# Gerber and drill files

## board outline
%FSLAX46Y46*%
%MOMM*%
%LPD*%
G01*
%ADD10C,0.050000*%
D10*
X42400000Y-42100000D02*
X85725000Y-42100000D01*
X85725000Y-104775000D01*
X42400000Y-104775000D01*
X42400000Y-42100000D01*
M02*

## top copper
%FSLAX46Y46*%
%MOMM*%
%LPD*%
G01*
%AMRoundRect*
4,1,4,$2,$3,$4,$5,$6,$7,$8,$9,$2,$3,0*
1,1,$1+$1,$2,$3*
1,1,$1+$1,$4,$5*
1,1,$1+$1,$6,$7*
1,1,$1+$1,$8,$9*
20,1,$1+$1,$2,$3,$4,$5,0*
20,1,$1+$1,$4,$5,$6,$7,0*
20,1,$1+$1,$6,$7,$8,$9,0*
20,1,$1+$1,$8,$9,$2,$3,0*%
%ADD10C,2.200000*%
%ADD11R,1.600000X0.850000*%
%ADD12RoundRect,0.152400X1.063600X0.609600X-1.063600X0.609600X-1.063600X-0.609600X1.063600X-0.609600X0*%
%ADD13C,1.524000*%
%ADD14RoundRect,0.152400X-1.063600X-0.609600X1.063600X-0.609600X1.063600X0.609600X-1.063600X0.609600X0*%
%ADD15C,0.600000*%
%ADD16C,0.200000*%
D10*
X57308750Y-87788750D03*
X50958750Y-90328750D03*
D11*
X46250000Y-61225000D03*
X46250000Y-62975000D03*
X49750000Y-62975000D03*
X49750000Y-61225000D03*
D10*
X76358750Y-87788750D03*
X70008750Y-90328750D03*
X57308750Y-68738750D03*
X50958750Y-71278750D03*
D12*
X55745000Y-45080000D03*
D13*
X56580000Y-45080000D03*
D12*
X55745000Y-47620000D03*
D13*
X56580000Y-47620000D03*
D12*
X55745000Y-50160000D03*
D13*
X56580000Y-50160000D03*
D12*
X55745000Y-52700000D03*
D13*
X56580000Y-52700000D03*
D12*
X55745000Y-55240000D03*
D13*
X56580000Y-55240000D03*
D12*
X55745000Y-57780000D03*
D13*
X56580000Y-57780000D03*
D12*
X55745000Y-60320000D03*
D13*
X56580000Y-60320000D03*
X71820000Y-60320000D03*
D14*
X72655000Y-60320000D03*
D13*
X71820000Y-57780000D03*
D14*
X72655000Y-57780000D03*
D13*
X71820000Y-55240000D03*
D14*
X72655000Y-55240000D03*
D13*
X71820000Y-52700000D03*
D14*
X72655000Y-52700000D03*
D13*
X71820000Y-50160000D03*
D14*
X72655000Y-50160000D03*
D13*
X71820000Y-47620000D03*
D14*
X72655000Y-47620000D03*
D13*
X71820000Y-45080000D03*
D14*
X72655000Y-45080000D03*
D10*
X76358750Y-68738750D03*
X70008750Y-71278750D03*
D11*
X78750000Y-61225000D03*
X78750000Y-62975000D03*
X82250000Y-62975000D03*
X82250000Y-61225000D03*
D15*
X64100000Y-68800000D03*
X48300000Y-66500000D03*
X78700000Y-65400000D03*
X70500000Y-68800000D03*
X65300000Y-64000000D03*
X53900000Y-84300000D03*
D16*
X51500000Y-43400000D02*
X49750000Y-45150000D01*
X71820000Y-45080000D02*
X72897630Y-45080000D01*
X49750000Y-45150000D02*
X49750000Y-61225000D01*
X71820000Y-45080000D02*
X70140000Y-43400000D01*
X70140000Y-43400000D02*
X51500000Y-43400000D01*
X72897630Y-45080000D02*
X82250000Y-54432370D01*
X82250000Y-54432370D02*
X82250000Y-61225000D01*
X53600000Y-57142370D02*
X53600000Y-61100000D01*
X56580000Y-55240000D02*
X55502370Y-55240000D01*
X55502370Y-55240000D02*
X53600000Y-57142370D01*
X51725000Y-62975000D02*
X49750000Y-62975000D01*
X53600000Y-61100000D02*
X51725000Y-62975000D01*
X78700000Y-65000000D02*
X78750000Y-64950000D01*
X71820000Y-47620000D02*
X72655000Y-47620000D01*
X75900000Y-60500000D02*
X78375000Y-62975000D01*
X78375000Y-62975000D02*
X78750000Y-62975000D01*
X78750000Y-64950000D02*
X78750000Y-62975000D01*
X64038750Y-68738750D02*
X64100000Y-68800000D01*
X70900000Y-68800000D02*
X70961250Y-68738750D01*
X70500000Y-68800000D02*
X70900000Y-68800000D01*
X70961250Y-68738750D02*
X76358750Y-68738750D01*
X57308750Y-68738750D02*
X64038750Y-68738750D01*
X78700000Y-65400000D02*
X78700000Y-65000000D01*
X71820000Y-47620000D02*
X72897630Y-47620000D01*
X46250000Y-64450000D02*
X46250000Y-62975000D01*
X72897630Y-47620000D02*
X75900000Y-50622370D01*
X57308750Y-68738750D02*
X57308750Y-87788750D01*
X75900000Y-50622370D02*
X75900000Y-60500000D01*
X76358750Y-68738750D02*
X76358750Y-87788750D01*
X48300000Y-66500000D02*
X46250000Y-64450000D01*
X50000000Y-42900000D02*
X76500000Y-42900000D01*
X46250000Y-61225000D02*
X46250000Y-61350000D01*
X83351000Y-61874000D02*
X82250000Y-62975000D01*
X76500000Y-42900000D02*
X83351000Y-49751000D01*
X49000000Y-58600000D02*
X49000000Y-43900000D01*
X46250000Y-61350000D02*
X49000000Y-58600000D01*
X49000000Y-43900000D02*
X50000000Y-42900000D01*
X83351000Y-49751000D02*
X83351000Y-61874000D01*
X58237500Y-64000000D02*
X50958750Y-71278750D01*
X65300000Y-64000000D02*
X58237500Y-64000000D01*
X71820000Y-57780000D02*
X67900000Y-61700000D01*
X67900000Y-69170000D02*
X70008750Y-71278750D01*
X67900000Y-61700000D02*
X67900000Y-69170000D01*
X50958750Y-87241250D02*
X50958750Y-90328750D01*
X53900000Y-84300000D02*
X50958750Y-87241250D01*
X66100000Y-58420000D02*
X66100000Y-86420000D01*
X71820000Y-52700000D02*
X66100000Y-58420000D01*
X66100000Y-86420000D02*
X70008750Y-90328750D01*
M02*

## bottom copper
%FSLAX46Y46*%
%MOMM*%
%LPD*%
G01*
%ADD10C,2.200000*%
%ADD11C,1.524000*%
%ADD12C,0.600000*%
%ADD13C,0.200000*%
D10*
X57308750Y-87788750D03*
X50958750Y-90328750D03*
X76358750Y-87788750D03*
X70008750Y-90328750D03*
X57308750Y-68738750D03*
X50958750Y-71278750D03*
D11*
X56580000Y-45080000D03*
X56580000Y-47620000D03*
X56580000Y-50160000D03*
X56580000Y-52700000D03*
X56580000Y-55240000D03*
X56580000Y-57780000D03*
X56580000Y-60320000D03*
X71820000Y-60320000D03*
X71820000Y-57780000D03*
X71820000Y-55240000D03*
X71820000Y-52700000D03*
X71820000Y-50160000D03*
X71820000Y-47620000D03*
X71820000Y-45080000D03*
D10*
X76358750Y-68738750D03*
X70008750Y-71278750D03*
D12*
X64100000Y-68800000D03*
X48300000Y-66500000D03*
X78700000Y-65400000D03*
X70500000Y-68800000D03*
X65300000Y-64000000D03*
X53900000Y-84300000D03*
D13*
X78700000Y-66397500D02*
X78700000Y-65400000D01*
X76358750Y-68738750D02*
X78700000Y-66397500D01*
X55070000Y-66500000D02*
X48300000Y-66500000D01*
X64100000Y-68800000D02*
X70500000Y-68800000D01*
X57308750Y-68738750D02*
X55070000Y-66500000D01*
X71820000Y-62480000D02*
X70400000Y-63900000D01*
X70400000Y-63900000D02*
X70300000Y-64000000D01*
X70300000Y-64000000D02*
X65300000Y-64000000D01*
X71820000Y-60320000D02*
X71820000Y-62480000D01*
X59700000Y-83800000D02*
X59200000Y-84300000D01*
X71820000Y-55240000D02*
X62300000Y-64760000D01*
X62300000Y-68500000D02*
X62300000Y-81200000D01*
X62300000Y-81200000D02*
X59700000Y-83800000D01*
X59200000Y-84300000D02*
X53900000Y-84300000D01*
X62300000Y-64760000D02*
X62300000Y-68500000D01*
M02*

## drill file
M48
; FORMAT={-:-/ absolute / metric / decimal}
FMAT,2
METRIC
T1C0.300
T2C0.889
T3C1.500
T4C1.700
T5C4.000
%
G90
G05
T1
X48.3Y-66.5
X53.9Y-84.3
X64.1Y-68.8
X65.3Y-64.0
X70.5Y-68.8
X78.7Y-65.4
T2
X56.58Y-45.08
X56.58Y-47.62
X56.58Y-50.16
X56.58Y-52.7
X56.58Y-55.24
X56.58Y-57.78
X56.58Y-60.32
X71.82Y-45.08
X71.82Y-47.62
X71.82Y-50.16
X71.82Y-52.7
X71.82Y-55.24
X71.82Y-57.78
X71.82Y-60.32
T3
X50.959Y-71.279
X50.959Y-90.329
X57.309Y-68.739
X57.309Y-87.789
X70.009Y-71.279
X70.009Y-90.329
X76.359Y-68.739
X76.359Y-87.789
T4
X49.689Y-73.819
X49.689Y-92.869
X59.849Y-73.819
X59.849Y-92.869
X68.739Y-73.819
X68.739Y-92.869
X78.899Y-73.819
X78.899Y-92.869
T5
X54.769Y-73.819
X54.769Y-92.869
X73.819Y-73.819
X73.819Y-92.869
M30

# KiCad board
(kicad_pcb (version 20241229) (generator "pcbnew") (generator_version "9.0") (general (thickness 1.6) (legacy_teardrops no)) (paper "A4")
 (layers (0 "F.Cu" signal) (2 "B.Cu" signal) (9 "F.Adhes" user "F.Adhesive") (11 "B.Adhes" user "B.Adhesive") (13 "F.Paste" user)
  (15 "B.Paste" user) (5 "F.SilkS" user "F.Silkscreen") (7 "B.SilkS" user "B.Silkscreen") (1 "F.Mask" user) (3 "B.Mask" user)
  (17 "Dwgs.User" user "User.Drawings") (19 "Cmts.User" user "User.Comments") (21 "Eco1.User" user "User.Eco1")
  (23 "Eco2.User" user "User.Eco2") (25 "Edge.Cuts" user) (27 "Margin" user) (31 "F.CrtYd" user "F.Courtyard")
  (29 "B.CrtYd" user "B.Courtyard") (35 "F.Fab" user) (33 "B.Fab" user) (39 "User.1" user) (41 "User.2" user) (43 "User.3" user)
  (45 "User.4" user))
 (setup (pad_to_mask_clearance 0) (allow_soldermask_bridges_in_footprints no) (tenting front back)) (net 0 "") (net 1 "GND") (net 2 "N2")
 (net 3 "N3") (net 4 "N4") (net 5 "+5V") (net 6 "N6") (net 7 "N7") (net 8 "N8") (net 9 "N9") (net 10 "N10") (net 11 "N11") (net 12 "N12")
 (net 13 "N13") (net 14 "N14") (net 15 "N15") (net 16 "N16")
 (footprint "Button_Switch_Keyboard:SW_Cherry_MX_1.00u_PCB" (layer "F.Cu") (at 57.30875 87.78875)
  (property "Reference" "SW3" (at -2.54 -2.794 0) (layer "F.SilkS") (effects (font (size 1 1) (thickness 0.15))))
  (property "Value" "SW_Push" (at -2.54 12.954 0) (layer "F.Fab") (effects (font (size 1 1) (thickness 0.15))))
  (pad "" np_thru_hole circle (at -7.62 5.08) (size 1.7 1.7) (drill 1.7) (layers "*.Cu" "*.Mask"))
  (pad "" np_thru_hole circle (at -2.54 5.08) (size 4 4) (drill 4) (layers "*.Cu" "*.Mask"))
  (pad "" np_thru_hole circle (at 2.54 5.08) (size 1.7 1.7) (drill 1.7) (layers "*.Cu" "*.Mask"))
  (pad "1" thru_hole circle (at 0 0) (size 2.2 2.2) (drill 1.5) (layers "*.Cu" "*.Mask") (remove_unused_layers no) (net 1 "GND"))
  (pad "2" thru_hole circle (at -6.35 2.54) (size 2.2 2.2) (drill 1.5) (layers "*.Cu" "*.Mask") (remove_unused_layers no) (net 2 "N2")))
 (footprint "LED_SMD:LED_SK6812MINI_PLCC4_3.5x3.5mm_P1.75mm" (layer "F.Cu") (at 48 62.1)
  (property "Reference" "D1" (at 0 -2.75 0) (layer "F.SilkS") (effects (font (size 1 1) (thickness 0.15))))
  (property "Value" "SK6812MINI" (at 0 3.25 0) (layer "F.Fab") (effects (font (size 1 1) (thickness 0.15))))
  (pad "1" smd rect (at -1.75 -0.875) (size 1.6 0.85) (layers "F.Cu" "F.Mask" "F.Paste") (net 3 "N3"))
  (pad "2" smd rect (at -1.75 0.875) (size 1.6 0.85) (layers "F.Cu" "F.Mask" "F.Paste") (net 1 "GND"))
  (pad "3" smd rect (at 1.75 0.875) (size 1.6 0.85) (layers "F.Cu" "F.Mask" "F.Paste") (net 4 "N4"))
  (pad "4" smd rect (at 1.75 -0.875) (size 1.6 0.85) (layers "F.Cu" "F.Mask" "F.Paste") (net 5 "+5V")))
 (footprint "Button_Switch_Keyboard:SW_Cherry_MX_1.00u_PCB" (layer "F.Cu") (at 76.35875 87.78875)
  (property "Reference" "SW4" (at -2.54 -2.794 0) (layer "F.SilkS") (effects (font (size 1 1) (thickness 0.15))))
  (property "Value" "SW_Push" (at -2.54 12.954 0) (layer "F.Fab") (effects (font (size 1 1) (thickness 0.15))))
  (pad "" np_thru_hole circle (at -7.62 5.08) (size 1.7 1.7) (drill 1.7) (layers "*.Cu" "*.Mask"))
  (pad "" np_thru_hole circle (at -2.54 5.08) (size 4 4) (drill 4) (layers "*.Cu" "*.Mask"))
  (pad "" np_thru_hole circle (at 2.54 5.08) (size 1.7 1.7) (drill 1.7) (layers "*.Cu" "*.Mask"))
  (pad "1" thru_hole circle (at 0 0) (size 2.2 2.2) (drill 1.5) (layers "*.Cu" "*.Mask") (remove_unused_layers no) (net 1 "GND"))
  (pad "2" thru_hole circle (at -6.35 2.54) (size 2.2 2.2) (drill 1.5) (layers "*.Cu" "*.Mask") (remove_unused_layers no) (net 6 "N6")))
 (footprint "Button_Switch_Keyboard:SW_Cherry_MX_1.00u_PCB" (layer "F.Cu") (at 57.30875 68.73875)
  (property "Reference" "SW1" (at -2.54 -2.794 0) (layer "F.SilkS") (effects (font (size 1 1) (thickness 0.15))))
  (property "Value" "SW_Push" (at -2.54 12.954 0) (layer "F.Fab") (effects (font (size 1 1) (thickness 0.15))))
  (pad "" np_thru_hole circle (at -7.62 5.08) (size 1.7 1.7) (drill 1.7) (layers "*.Cu" "*.Mask"))
  (pad "" np_thru_hole circle (at -2.54 5.08) (size 4 4) (drill 4) (layers "*.Cu" "*.Mask"))
  (pad "" np_thru_hole circle (at 2.54 5.08) (size 1.7 1.7) (drill 1.7) (layers "*.Cu" "*.Mask"))
  (pad "1" thru_hole circle (at 0 0) (size 2.2 2.2) (drill 1.5) (layers "*.Cu" "*.Mask") (remove_unused_layers no) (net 1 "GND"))
  (pad "2" thru_hole circle (at -6.35 2.54) (size 2.2 2.2) (drill 1.5) (layers "*.Cu" "*.Mask") (remove_unused_layers no) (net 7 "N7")))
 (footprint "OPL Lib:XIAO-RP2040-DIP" (layer "F.Cu") (at 64.2 52.7)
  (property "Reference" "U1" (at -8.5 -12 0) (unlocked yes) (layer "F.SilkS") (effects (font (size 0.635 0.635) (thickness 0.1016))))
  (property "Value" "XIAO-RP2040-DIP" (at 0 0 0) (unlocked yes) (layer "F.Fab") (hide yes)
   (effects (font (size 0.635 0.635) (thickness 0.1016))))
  (pad "1" smd roundrect (at -8.455 -7.62 180) (size 2.432 1.524) (layers "F.Cu" "F.Mask") (roundrect_rratio 0.1) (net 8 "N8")
   (thermal_bridge_angle 45))
  (pad "1" thru_hole circle (at -7.62 -7.62 180) (size 1.524 1.524) (drill 0.889) (layers "*.Cu" "*.Mask") (remove_unused_layers no)
   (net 8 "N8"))
  (pad "2" smd roundrect (at -8.455 -5.08 180) (size 2.432 1.524) (layers "F.Cu" "F.Mask") (roundrect_rratio 0.1) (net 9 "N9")
   (thermal_bridge_angle 45))
  (pad "2" thru_hole circle (at -7.62 -5.08 180) (size 1.524 1.524) (drill 0.889) (layers "*.Cu" "*.Mask") (remove_unused_layers no)
   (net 9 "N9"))
  (pad "3" smd roundrect (at -8.455 -2.54 180) (size 2.432 1.524) (layers "F.Cu" "F.Mask") (roundrect_rratio 0.1) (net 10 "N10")
   (thermal_bridge_angle 45))
  (pad "3" thru_hole circle (at -7.62 -2.54 180) (size 1.524 1.524) (drill 0.889) (layers "*.Cu" "*.Mask") (remove_unused_layers no)
   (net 10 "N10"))
  (pad "4" smd roundrect (at -8.455 0 180) (size 2.432 1.524) (layers "F.Cu" "F.Mask") (roundrect_rratio 0.1) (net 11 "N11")
   (thermal_bridge_angle 45))
  (pad "4" thru_hole circle (at -7.62 0 180) (size 1.524 1.524) (drill 0.889) (layers "*.Cu" "*.Mask") (remove_unused_layers no)
   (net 11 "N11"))
  (pad "5" smd roundrect (at -8.455 2.54 180) (size 2.432 1.524) (layers "F.Cu" "F.Mask") (roundrect_rratio 0.1) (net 4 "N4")
   (thermal_bridge_angle 45))
  (pad "5" thru_hole circle (at -7.62 2.54 180) (size 1.524 1.524) (drill 0.889) (layers "*.Cu" "*.Mask") (remove_unused_layers no)
   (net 4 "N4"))
  (pad "6" smd roundrect (at -8.455 5.08 180) (size 2.432 1.524) (layers "F.Cu" "F.Mask") (roundrect_rratio 0.1) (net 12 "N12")
   (thermal_bridge_angle 45))
  (pad "6" thru_hole circle (at -7.62 5.08 180) (size 1.524 1.524) (drill 0.889) (layers "*.Cu" "*.Mask") (remove_unused_layers no)
   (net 12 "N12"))
  (pad "7" smd roundrect (at -8.455 7.62 180) (size 2.432 1.524) (layers "F.Cu" "F.Mask") (roundrect_rratio 0.1) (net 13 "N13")
   (thermal_bridge_angle 45))
  (pad "7" thru_hole circle (at -7.62 7.62 180) (size 1.524 1.524) (drill 0.889) (layers "*.Cu" "*.Mask") (remove_unused_layers no)
   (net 13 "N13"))
  (pad "8" thru_hole circle (at 7.62 7.62) (size 1.524 1.524) (drill 0.889) (layers "*.Cu" "*.Mask") (remove_unused_layers no) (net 7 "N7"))
  (pad "8" smd roundrect (at 8.455 7.62) (size 2.432 1.524) (layers "F.Cu" "F.Mask") (roundrect_rratio 0.1) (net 7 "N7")
   (thermal_bridge_angle 45))
  (pad "9" thru_hole circle (at 7.62 5.08) (size 1.524 1.524) (drill 0.889) (layers "*.Cu" "*.Mask") (remove_unused_layers no)
   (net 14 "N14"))
  (pad "9" smd roundrect (at 8.455 5.08) (size 2.432 1.524) (layers "F.Cu" "F.Mask") (roundrect_rratio 0.1) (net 14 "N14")
   (thermal_bridge_angle 45))
  (pad "10" thru_hole circle (at 7.62 2.54) (size 1.524 1.524) (drill 0.889) (layers "*.Cu" "*.Mask") (remove_unused_layers no) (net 2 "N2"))
  (pad "10" smd roundrect (at 8.455 2.54) (size 2.432 1.524) (layers "F.Cu" "F.Mask") (roundrect_rratio 0.1) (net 2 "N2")
   (thermal_bridge_angle 45))
  (pad "11" thru_hole circle (at 7.62 0) (size 1.524 1.524) (drill 0.889) (layers "*.Cu" "*.Mask") (remove_unused_layers no) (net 6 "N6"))
  (pad "11" smd roundrect (at 8.455 0) (size 2.432 1.524) (layers "F.Cu" "F.Mask") (roundrect_rratio 0.1) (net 6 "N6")
   (thermal_bridge_angle 45))
  (pad "12" thru_hole circle (at 7.62 -2.54) (size 1.524 1.524) (drill 0.889) (layers "*.Cu" "*.Mask") (remove_unused_layers no)
   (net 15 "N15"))
  (pad "12" smd roundrect (at 8.455 -2.54) (size 2.432 1.524) (layers "F.Cu" "F.Mask") (roundrect_rratio 0.1) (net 15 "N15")
   (thermal_bridge_angle 45))
  (pad "13" thru_hole circle (at 7.62 -5.08) (size 1.524 1.524) (drill 0.889) (layers "*.Cu" "*.Mask") (remove_unused_layers no)
   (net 1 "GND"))
  (pad "13" smd roundrect (at 8.455 -5.08) (size 2.432 1.524) (layers "F.Cu" "F.Mask") (roundrect_rratio 0.1) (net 1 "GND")
   (thermal_bridge_angle 45))
  (pad "14" thru_hole circle (at 7.62 -7.62) (size 1.524 1.524) (drill 0.889) (layers "*.Cu" "*.Mask") (remove_unused_layers no)
   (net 5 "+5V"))
  (pad "14" smd roundrect (at 8.455 -7.62) (size 2.432 1.524) (layers "F.Cu" "F.Mask") (roundrect_rratio 0.1) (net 5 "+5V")
   (thermal_bridge_angle 45)))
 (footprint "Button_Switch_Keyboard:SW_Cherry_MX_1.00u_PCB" (layer "F.Cu") (at 76.35875 68.73875)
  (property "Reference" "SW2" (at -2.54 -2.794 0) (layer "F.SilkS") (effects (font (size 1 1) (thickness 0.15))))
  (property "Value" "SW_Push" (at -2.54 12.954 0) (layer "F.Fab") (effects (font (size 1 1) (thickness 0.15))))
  (pad "" np_thru_hole circle (at -7.62 5.08) (size 1.7 1.7) (drill 1.7) (layers "*.Cu" "*.Mask"))
  (pad "" np_thru_hole circle (at -2.54 5.08) (size 4 4) (drill 4) (layers "*.Cu" "*.Mask"))
  (pad "" np_thru_hole circle (at 2.54 5.08) (size 1.7 1.7) (drill 1.7) (layers "*.Cu" "*.Mask"))
  (pad "1" thru_hole circle (at 0 0) (size 2.2 2.2) (drill 1.5) (layers "*.Cu" "*.Mask") (remove_unused_layers no) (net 1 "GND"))
  (pad "2" thru_hole circle (at -6.35 2.54) (size 2.2 2.2) (drill 1.5) (layers "*.Cu" "*.Mask") (remove_unused_layers no) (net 14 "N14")))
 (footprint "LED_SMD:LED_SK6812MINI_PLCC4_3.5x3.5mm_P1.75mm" (layer "F.Cu") (at 80.5 62.1)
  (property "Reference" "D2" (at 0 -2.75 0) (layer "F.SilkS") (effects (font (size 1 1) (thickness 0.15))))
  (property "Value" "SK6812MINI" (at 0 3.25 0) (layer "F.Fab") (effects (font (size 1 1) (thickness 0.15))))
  (pad "1" smd rect (at -1.75 -0.875) (size 1.6 0.85) (layers "F.Cu" "F.Mask" "F.Paste") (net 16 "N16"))
  (pad "2" smd rect (at -1.75 0.875) (size 1.6 0.85) (layers "F.Cu" "F.Mask" "F.Paste") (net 1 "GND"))
  (pad "3" smd rect (at 1.75 0.875) (size 1.6 0.85) (layers "F.Cu" "F.Mask" "F.Paste") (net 3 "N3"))
  (pad "4" smd rect (at 1.75 -0.875) (size 1.6 0.85) (layers "F.Cu" "F.Mask" "F.Paste") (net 5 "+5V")))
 (gr_rect (start 42.4 42.1) (end 85.725 104.775) (stroke (width 0.05) (type default)) (fill no) (layer "Edge.Cuts"))
 (segment (start 51.5 43.4) (end 49.75 45.15) (width 0.2) (layer "F.Cu") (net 5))
 (segment (start 71.82 45.08) (end 72.89763 45.08) (width 0.2) (layer "F.Cu") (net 5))
 (segment (start 49.75 45.15) (end 49.75 61.225) (width 0.2) (layer "F.Cu") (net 5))
 (segment (start 71.82 45.08) (end 70.14 43.4) (width 0.2) (layer "F.Cu") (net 5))
 (segment (start 70.14 43.4) (end 51.5 43.4) (width 0.2) (layer "F.Cu") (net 5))
 (segment (start 72.89763 45.08) (end 82.25 54.43237) (width 0.2) (layer "F.Cu") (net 5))
 (segment (start 82.25 54.43237) (end 82.25 61.225) (width 0.2) (layer "F.Cu") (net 5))
 (segment (start 53.6 57.14237) (end 53.6 61.1) (width 0.2) (layer "F.Cu") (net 4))
 (segment (start 56.58 55.24) (end 55.50237 55.24) (width 0.2) (layer "F.Cu") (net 4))
 (segment (start 55.50237 55.24) (end 53.6 57.14237) (width 0.2) (layer "F.Cu") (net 4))
 (segment (start 51.725 62.975) (end 49.75 62.975) (width 0.2) (layer "F.Cu") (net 4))
 (segment (start 53.6 61.1) (end 51.725 62.975) (width 0.2) (layer "F.Cu") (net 4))
 (segment (start 78.7 65) (end 78.75 64.95) (width 0.2) (layer "F.Cu") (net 1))
 (segment (start 71.82 47.62) (end 72.655 47.62) (width 0.2) (layer "F.Cu") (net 1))
 (segment (start 75.9 60.5) (end 78.375 62.975) (width 0.2) (layer "F.Cu") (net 1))
 (segment (start 78.375 62.975) (end 78.75 62.975) (width 0.2) (layer "F.Cu") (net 1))
 (segment (start 78.75 64.95) (end 78.75 62.975) (width 0.2) (layer "F.Cu") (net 1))
 (segment (start 64.03875 68.73875) (end 64.1 68.8) (width 0.2) (layer "F.Cu") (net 1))
 (segment (start 70.9 68.8) (end 70.96125 68.73875) (width 0.2) (layer "F.Cu") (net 1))
 (segment (start 70.5 68.8) (end 70.9 68.8) (width 0.2) (layer "F.Cu") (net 1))
 (segment (start 70.96125 68.73875) (end 76.35875 68.73875) (width 0.2) (layer "F.Cu") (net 1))
 (segment (start 57.30875 68.73875) (end 64.03875 68.73875) (width 0.2) (layer "F.Cu") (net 1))
 (segment (start 78.7 65.4) (end 78.7 65) (width 0.2) (layer "F.Cu") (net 1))
 (segment (start 71.82 47.62) (end 72.89763 47.62) (width 0.2) (layer "F.Cu") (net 1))
 (segment (start 46.25 64.45) (end 46.25 62.975) (width 0.2) (layer "F.Cu") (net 1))
 (segment (start 72.89763 47.62) (end 75.9 50.62237) (width 0.2) (layer "F.Cu") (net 1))
 (segment (start 57.30875 68.73875) (end 57.30875 87.78875) (width 0.2) (layer "F.Cu") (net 1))
 (segment (start 75.9 50.62237) (end 75.9 60.5) (width 0.2) (layer "F.Cu") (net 1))
 (segment (start 76.35875 68.73875) (end 76.35875 87.78875) (width 0.2) (layer "F.Cu") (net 1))
 (segment (start 48.3 66.5) (end 46.25 64.45) (width 0.2) (layer "F.Cu") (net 1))
 (via (at 64.1 68.8) (size 0.6) (drill 0.3) (layers "F.Cu" "B.Cu") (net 1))
 (via (at 48.3 66.5) (size 0.6) (drill 0.3) (layers "F.Cu" "B.Cu") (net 1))
 (via (at 78.7 65.4) (size 0.6) (drill 0.3) (layers "F.Cu" "B.Cu") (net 1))
 (via (at 70.5 68.8) (size 0.6) (drill 0.3) (layers "F.Cu" "B.Cu") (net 1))
 (segment (start 78.7 66.3975) (end 78.7 65.4) (width 0.2) (layer "B.Cu") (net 1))
 (segment (start 76.35875 68.73875) (end 78.7 66.3975) (width 0.2) (layer "B.Cu") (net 1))
 (segment (start 55.07 66.5) (end 48.3 66.5) (width 0.2) (layer "B.Cu") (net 1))
 (segment (start 64.1 68.8) (end 70.5 68.8) (width 0.2) (layer "B.Cu") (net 1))
 (segment (start 57.30875 68.73875) (end 55.07 66.5) (width 0.2) (layer "B.Cu") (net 1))
 (segment (start 50 42.9) (end 76.5 42.9) (width 0.2) (layer "F.Cu") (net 3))
 (segment (start 46.25 61.225) (end 46.25 61.35) (width 0.2) (layer "F.Cu") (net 3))
 (segment (start 83.351 61.874) (end 82.25 62.975) (width 0.2) (layer "F.Cu") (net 3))
 (segment (start 76.5 42.9) (end 83.351 49.751) (width 0.2) (layer "F.Cu") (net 3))
 (segment (start 49 58.6) (end 49 43.9) (width 0.2) (layer "F.Cu") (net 3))
 (segment (start 46.25 61.35) (end 49 58.6) (width 0.2) (layer "F.Cu") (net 3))
 (segment (start 49 43.9) (end 50 42.9) (width 0.2) (layer "F.Cu") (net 3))
 (segment (start 83.351 49.751) (end 83.351 61.874) (width 0.2) (layer "F.Cu") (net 3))
 (segment (start 58.2375 64) (end 50.95875 71.27875) (width 0.2) (layer "F.Cu") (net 7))
 (segment (start 65.3 64) (end 58.2375 64) (width 0.2) (layer "F.Cu") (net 7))
 (via (at 65.3 64) (size 0.6) (drill 0.3) (layers "F.Cu" "B.Cu") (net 7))
 (segment (start 71.82 62.48) (end 70.4 63.9) (width 0.2) (layer "B.Cu") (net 7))
 (segment (start 70.4 63.9) (end 70.3 64) (width 0.2) (layer "B.Cu") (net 7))
 (segment (start 70.3 64) (end 65.3 64) (width 0.2) (layer "B.Cu") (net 7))
 (segment (start 71.82 60.32) (end 71.82 62.48) (width 0.2) (layer "B.Cu") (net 7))
 (segment (start 71.82 57.78) (end 67.9 61.7) (width 0.2) (layer "F.Cu") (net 14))
 (segment (start 67.9 69.17) (end 70.00875 71.27875) (width 0.2) (layer "F.Cu") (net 14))
 (segment (start 67.9 61.7) (end 67.9 69.17) (width 0.2) (layer "F.Cu") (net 14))
 (segment (start 50.95875 87.24125) (end 50.95875 90.32875) (width 0.2) (layer "F.Cu") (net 2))
 (segment (start 53.9 84.3) (end 50.95875 87.24125) (width 0.2) (layer "F.Cu") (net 2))
 (via (at 53.9 84.3) (size 0.6) (drill 0.3) (layers "F.Cu" "B.Cu") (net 2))
 (segment (start 59.7 83.8) (end 59.2 84.3) (width 0.2) (layer "B.Cu") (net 2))
 (segment (start 71.82 55.24) (end 62.3 64.76) (width 0.2) (layer "B.Cu") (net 2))
 (segment (start 62.3 68.5) (end 62.3 81.2) (width 0.2) (layer "B.Cu") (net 2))
 (segment (start 62.3 81.2) (end 59.7 83.8) (width 0.2) (layer "B.Cu") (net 2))
 (segment (start 59.2 84.3) (end 53.9 84.3) (width 0.2) (layer "B.Cu") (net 2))
 (segment (start 62.3 64.76) (end 62.3 68.5) (width 0.2) (layer "B.Cu") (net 2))
 (segment (start 66.1 58.42) (end 66.1 86.42) (width 0.2) (layer "F.Cu") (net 6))
 (segment (start 71.82 52.7) (end 66.1 58.42) (width 0.2) (layer "F.Cu") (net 6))
 (segment (start 66.1 86.42) (end 70.00875 90.32875) (width 0.2) (layer "F.Cu") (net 6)))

